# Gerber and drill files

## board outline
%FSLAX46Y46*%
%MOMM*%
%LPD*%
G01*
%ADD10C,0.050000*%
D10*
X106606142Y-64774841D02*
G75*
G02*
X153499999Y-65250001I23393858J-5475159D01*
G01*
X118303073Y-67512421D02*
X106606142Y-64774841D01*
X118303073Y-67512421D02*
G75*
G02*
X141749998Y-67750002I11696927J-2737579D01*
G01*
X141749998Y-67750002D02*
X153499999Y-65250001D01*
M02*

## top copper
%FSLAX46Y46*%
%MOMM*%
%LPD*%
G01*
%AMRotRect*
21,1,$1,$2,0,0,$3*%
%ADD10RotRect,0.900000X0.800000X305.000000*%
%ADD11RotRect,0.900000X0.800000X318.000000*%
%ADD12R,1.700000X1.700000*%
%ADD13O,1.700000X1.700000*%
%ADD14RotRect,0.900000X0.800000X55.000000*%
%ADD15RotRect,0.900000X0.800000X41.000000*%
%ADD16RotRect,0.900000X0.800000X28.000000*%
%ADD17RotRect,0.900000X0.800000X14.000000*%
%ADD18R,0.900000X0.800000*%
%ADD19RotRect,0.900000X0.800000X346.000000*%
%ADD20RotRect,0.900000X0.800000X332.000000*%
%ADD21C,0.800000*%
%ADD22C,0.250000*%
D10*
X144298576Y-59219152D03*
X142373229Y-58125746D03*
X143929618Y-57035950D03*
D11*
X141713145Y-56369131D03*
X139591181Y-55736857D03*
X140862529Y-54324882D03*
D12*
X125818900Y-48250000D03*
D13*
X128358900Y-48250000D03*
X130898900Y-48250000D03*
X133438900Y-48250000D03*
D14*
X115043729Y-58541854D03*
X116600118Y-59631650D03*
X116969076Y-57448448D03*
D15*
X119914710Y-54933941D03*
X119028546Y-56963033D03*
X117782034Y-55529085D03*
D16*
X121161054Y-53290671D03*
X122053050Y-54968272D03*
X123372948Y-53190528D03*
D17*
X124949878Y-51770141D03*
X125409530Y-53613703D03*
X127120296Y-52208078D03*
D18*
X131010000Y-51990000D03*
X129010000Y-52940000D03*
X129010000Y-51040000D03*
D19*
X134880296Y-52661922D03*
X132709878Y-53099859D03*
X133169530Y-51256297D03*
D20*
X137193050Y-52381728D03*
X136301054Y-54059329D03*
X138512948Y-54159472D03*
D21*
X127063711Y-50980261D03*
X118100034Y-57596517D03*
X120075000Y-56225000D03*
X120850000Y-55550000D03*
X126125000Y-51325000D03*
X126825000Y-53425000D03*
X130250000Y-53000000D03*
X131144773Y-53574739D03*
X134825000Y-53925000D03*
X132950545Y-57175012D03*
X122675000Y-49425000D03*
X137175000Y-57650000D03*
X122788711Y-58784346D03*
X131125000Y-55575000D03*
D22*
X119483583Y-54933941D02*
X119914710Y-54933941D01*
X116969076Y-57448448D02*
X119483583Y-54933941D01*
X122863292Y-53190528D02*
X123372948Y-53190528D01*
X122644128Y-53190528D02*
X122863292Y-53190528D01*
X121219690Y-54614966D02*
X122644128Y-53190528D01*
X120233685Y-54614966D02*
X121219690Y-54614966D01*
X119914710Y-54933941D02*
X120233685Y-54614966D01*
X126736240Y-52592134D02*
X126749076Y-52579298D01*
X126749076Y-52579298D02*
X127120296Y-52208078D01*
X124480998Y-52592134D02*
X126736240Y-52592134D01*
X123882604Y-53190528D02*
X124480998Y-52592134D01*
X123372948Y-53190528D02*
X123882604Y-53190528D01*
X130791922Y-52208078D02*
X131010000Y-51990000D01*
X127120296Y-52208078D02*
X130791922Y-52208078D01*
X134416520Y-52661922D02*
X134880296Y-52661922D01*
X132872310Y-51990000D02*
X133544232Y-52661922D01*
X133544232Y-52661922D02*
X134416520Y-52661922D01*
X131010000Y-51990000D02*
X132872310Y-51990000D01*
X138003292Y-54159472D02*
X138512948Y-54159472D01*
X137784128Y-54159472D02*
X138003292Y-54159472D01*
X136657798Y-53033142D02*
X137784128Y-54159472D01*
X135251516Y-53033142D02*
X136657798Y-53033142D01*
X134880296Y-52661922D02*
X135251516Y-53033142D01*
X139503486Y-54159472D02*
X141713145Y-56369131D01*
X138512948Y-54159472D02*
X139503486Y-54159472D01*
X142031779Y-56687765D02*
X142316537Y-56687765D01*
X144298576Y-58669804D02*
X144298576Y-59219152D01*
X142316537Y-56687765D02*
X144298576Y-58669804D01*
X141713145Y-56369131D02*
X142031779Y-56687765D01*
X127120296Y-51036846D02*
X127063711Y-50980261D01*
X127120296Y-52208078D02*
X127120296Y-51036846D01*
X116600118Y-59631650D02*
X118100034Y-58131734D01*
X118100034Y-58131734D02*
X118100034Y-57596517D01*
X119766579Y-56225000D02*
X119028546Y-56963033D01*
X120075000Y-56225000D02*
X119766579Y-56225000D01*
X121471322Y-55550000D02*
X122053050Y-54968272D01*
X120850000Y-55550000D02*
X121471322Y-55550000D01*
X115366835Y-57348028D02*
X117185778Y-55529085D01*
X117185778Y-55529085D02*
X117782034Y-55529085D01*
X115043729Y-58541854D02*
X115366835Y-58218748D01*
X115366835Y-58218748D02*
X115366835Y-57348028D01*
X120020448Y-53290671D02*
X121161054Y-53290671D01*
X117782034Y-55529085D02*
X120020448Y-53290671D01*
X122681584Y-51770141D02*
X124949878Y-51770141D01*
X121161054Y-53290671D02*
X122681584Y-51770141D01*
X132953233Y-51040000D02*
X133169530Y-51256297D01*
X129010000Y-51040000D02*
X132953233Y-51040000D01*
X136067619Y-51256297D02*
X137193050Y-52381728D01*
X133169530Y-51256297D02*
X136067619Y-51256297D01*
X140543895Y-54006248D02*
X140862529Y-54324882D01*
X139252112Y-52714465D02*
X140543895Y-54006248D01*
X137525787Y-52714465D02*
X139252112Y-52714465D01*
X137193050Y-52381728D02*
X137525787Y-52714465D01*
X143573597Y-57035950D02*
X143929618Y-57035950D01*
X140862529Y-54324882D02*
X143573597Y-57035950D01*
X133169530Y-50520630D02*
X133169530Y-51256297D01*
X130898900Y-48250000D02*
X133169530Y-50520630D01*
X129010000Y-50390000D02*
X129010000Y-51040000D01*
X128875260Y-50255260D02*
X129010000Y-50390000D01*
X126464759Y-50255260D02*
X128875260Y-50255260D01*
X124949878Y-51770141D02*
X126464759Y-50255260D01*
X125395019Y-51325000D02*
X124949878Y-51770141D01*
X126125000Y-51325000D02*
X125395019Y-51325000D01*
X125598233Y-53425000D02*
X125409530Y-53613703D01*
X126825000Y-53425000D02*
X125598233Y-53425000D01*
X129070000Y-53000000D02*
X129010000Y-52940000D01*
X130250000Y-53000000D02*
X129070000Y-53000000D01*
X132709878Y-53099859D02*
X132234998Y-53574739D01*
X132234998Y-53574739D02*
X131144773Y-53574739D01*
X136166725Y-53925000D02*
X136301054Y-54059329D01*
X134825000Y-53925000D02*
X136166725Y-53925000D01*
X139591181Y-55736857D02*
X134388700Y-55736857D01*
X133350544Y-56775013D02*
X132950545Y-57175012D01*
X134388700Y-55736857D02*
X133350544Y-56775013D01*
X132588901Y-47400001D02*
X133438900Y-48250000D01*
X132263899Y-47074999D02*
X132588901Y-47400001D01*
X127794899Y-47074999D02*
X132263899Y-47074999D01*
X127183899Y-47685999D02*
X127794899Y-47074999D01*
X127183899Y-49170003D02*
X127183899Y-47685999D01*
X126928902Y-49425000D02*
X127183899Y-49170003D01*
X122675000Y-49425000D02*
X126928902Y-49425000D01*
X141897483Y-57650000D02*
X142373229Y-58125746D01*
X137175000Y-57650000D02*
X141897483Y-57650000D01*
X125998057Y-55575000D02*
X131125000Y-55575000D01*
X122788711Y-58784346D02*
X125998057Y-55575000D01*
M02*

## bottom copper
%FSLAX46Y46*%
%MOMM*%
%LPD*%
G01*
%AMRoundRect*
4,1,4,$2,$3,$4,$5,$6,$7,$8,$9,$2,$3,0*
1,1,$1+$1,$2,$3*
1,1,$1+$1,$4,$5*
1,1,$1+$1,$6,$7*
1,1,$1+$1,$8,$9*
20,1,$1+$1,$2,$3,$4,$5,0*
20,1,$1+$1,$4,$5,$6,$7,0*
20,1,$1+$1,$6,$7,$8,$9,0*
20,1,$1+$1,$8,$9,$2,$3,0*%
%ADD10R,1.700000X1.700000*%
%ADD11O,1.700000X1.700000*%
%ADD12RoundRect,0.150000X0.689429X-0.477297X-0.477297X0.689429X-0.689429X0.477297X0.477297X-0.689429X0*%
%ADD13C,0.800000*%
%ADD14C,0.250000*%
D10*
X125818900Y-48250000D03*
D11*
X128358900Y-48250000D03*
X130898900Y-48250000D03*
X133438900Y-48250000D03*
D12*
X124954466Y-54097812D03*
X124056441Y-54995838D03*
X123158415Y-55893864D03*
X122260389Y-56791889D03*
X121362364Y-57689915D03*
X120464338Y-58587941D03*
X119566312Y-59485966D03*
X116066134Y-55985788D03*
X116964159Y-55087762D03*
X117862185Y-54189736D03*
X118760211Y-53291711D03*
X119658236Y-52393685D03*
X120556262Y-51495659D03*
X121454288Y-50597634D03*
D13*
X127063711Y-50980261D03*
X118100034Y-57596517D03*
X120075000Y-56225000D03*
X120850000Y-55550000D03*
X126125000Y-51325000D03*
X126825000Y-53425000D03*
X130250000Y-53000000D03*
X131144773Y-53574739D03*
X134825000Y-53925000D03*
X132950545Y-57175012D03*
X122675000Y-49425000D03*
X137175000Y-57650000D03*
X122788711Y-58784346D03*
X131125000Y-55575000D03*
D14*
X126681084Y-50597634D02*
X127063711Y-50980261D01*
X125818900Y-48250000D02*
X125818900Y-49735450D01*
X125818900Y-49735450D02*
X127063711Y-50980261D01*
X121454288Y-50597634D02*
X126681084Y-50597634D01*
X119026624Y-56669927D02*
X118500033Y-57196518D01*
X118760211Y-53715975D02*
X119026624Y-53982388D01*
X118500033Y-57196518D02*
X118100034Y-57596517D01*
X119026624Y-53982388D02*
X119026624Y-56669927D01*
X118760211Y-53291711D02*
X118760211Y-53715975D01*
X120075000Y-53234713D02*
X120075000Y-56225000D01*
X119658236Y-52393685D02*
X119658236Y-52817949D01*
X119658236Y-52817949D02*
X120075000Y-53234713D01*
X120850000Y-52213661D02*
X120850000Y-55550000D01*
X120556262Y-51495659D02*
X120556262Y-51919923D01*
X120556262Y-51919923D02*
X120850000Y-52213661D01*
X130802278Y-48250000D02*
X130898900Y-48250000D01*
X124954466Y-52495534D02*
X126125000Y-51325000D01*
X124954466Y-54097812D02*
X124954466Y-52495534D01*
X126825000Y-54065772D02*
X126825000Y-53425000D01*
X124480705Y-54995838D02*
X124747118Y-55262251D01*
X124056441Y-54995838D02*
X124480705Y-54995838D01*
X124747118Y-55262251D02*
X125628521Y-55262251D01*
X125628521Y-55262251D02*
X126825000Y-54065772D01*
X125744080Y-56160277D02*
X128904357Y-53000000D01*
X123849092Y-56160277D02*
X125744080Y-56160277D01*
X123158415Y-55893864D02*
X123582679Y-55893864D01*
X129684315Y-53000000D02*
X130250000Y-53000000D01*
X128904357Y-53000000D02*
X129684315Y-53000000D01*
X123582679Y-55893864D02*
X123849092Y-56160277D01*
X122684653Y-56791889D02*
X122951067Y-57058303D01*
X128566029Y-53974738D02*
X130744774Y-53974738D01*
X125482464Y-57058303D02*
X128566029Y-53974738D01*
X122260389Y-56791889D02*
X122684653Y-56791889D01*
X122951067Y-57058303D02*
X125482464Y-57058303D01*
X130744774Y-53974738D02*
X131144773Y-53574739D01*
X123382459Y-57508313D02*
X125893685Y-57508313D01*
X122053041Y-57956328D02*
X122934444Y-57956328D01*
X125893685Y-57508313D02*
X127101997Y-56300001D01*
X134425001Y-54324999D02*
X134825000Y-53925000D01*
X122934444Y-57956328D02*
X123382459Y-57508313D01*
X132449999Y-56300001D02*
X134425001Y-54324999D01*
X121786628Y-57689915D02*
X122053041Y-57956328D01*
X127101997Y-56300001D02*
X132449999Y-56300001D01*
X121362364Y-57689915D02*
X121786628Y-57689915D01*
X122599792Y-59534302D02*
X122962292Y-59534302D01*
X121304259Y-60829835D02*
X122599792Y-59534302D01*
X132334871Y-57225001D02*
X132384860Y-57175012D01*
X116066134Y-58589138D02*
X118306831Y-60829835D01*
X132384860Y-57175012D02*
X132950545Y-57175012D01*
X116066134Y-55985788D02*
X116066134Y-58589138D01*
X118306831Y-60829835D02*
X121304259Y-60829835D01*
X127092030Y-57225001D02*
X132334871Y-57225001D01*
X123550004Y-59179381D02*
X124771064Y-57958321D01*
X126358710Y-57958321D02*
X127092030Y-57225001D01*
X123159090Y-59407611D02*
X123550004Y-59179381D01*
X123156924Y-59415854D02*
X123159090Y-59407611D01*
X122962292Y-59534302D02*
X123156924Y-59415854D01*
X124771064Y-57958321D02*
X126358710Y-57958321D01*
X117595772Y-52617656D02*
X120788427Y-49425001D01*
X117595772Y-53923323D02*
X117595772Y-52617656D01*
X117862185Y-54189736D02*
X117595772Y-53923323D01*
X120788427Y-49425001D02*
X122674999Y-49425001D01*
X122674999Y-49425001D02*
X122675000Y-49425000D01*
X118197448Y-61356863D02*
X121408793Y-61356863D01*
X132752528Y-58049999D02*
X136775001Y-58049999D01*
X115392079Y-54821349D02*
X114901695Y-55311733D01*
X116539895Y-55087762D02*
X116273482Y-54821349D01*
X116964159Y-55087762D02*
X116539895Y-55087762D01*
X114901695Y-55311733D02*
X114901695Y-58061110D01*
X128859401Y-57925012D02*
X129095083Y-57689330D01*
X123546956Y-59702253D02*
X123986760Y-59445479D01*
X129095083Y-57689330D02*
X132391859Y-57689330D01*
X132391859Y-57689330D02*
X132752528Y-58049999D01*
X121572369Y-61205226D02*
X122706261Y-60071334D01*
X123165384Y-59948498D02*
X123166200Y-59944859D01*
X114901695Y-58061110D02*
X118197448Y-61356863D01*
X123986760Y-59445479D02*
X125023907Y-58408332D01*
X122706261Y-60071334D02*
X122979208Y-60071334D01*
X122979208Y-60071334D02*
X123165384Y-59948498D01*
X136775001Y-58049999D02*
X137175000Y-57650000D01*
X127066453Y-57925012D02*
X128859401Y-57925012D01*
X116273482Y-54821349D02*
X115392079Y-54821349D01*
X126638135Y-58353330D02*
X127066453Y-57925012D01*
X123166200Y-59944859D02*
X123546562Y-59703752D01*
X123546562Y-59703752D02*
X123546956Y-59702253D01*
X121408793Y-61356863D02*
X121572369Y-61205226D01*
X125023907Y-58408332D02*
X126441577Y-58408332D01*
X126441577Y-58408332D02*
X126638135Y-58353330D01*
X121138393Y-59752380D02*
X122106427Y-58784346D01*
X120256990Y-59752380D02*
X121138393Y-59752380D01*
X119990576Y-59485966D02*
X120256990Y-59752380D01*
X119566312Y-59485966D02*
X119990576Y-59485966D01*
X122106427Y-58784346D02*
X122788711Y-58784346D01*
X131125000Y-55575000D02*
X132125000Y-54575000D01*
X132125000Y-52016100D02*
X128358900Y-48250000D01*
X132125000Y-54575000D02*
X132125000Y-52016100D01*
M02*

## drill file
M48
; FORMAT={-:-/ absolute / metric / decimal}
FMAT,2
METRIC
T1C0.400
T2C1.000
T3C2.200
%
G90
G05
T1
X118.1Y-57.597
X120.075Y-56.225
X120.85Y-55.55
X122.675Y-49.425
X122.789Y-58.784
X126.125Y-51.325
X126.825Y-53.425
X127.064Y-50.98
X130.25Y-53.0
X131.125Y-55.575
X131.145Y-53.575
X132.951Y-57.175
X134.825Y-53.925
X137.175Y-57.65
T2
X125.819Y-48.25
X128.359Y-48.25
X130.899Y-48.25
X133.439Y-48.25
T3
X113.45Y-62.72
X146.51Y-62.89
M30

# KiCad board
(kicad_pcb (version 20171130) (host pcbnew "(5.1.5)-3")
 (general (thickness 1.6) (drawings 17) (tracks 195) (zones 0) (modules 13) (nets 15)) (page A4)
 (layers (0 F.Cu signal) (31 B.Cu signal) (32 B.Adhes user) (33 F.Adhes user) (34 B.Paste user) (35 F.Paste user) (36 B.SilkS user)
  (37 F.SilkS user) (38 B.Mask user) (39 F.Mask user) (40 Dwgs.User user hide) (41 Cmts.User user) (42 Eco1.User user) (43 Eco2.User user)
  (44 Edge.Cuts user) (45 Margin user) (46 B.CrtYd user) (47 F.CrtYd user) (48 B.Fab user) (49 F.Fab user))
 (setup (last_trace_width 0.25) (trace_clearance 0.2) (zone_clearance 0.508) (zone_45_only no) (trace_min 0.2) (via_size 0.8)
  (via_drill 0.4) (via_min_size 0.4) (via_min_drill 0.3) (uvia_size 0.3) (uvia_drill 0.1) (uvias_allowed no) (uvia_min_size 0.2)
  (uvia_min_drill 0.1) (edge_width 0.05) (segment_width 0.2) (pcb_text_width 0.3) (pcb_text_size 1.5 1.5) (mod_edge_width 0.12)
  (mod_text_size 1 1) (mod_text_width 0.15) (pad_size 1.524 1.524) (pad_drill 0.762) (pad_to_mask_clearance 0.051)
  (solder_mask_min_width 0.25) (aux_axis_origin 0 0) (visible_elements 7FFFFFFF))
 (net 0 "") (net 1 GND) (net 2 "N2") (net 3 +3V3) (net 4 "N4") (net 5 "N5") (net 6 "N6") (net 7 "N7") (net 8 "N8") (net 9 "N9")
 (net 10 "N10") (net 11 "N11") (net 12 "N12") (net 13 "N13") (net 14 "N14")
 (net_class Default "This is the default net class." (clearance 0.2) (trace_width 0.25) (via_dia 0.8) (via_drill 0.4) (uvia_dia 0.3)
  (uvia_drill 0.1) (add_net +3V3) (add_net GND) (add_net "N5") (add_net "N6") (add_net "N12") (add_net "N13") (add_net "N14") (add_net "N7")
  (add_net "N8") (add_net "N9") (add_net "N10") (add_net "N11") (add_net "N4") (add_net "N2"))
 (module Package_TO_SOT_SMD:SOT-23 (layer F.Cu) (at 143.725 58.4 305)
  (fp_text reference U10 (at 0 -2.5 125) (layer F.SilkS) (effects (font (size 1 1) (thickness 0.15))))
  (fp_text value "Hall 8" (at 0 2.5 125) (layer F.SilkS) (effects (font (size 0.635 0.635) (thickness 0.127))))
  (pad 3 smd rect (at 1 0 305) (size 0.9 0.8) (layers F.Cu F.Paste F.Mask) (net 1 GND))
  (pad 2 smd rect (at -1 0.95 305) (size 0.9 0.8) (layers F.Cu F.Paste F.Mask) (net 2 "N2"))
  (pad 1 smd rect (at -1 -0.95 305) (size 0.9 0.8) (layers F.Cu F.Paste F.Mask) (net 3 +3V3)))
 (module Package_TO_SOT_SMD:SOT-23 (layer F.Cu) (at 140.97 55.7 318)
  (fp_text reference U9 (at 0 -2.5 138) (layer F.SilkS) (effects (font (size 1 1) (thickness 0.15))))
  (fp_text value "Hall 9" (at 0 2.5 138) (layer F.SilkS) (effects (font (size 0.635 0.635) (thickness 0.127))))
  (pad 3 smd rect (at 1 0 318) (size 0.9 0.8) (layers F.Cu F.Paste F.Mask) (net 1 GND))
  (pad 2 smd rect (at -1 0.95 318) (size 0.9 0.8) (layers F.Cu F.Paste F.Mask) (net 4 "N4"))
  (pad 1 smd rect (at -1 -0.95 318) (size 0.9 0.8) (layers F.Cu F.Paste F.Mask) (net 3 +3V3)))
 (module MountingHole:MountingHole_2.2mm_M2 (layer F.Cu) (at 146.51 62.89)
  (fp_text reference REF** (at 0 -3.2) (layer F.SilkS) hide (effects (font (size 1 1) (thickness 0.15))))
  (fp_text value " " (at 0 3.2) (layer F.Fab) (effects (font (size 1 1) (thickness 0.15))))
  (pad 1 np_thru_hole circle (at 0 0) (size 2.2 2.2) (drill 2.2) (layers *.Cu *.Mask)))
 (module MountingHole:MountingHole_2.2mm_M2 (layer F.Cu) (at 113.45 62.72)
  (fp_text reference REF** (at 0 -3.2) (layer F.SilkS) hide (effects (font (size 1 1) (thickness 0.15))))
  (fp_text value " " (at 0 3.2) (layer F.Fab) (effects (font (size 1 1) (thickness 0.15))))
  (pad 1 np_thru_hole circle (at 0 0) (size 2.2 2.2) (drill 2.2) (layers *.Cu *.Mask)))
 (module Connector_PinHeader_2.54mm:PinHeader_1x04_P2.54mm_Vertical (layer F.Cu) (at 125.8189 48.25 90)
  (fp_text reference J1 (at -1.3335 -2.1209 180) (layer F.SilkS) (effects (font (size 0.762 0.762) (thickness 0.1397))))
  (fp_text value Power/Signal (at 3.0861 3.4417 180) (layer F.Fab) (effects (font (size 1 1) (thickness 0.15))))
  (pad 1 thru_hole rect (at 0 0 90) (size 1.7 1.7) (drill 1) (layers *.Cu *.Mask) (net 1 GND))
  (pad 2 thru_hole oval (at 0 2.54 90) (size 1.7 1.7) (drill 1) (layers *.Cu *.Mask) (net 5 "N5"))
  (pad 3 thru_hole oval (at 0 5.08 90) (size 1.7 1.7) (drill 1) (layers *.Cu *.Mask) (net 3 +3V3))
  (pad 4 thru_hole oval (at 0 7.62 90) (size 1.7 1.7) (drill 1) (layers *.Cu *.Mask) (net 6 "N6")))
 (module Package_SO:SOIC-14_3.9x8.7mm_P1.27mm (layer B.Cu) (at 120.5103 55.0418 135)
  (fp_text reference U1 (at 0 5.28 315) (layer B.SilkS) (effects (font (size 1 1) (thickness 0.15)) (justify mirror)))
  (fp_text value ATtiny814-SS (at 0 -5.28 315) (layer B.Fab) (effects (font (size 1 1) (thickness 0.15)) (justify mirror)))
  (pad 1 smd roundrect (at -2.475 3.81 135) (size 1.95 0.6) (layers B.Cu B.Paste B.Mask) (roundrect_rratio 0.25) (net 3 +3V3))
  (pad 2 smd roundrect (at -2.475 2.54 135) (size 1.95 0.6) (layers B.Cu B.Paste B.Mask) (roundrect_rratio 0.25) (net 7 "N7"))
  (pad 3 smd roundrect (at -2.475 1.27 135) (size 1.95 0.6) (layers B.Cu B.Paste B.Mask) (roundrect_rratio 0.25) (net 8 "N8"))
  (pad 4 smd roundrect (at -2.475 0 135) (size 1.95 0.6) (layers B.Cu B.Paste B.Mask) (roundrect_rratio 0.25) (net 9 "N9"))
  (pad 5 smd roundrect (at -2.475 -1.27 135) (size 1.95 0.6) (layers B.Cu B.Paste B.Mask) (roundrect_rratio 0.25) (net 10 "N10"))
  (pad 6 smd roundrect (at -2.475 -2.54 135) (size 1.95 0.6) (layers B.Cu B.Paste B.Mask) (roundrect_rratio 0.25) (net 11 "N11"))
  (pad 7 smd roundrect (at -2.475 -3.81 135) (size 1.95 0.6) (layers B.Cu B.Paste B.Mask) (roundrect_rratio 0.25) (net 5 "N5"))
  (pad 8 smd roundrect (at 2.475 -3.81 135) (size 1.95 0.6) (layers B.Cu B.Paste B.Mask) (roundrect_rratio 0.25) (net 4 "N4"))
  (pad 9 smd roundrect (at 2.475 -2.54 135) (size 1.95 0.6) (layers B.Cu B.Paste B.Mask) (roundrect_rratio 0.25) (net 2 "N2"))
  (pad 10 smd roundrect (at 2.475 -1.27 135) (size 1.95 0.6) (layers B.Cu B.Paste B.Mask) (roundrect_rratio 0.25) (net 6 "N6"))
  (pad 11 smd roundrect (at 2.475 0 135) (size 1.95 0.6) (layers B.Cu B.Paste B.Mask) (roundrect_rratio 0.25) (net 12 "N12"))
  (pad 12 smd roundrect (at 2.475 1.27 135) (size 1.95 0.6) (layers B.Cu B.Paste B.Mask) (roundrect_rratio 0.25) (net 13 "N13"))
  (pad 13 smd roundrect (at 2.475 2.54 135) (size 1.95 0.6) (layers B.Cu B.Paste B.Mask) (roundrect_rratio 0.25) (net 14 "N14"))
  (pad 14 smd roundrect (at 2.475 3.81 135) (size 1.95 0.6) (layers B.Cu B.Paste B.Mask) (roundrect_rratio 0.25) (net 1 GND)))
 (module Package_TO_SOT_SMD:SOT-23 (layer F.Cu) (at 116.3955 58.2676 55)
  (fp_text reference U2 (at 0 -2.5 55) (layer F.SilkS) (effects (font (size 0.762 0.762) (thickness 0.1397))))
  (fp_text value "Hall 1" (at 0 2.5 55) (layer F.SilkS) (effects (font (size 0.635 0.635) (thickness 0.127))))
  (pad 1 smd rect (at -1 -0.95 55) (size 0.9 0.8) (layers F.Cu F.Paste F.Mask) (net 3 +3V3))
  (pad 2 smd rect (at -1 0.95 55) (size 0.9 0.8) (layers F.Cu F.Paste F.Mask) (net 12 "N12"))
  (pad 3 smd rect (at 1 0 55) (size 0.9 0.8) (layers F.Cu F.Paste F.Mask) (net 1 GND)))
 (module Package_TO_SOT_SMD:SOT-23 (layer F.Cu) (at 119.16 55.59 41)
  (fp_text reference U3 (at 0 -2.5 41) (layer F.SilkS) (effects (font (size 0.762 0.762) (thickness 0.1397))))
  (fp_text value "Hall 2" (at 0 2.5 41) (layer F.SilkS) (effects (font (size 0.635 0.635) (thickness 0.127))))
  (pad 3 smd rect (at 1 0 41) (size 0.9 0.8) (layers F.Cu F.Paste F.Mask) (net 1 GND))
  (pad 2 smd rect (at -1 0.95 41) (size 0.9 0.8) (layers F.Cu F.Paste F.Mask) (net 13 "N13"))
  (pad 1 smd rect (at -1 -0.95 41) (size 0.9 0.8) (layers F.Cu F.Paste F.Mask) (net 3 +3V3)))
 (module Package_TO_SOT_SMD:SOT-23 (layer F.Cu) (at 122.49 53.66 28)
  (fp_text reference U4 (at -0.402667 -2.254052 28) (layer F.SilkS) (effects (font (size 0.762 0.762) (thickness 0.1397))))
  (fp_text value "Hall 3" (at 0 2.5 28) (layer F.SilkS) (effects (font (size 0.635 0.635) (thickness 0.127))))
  (pad 1 smd rect (at -1 -0.95 28) (size 0.9 0.8) (layers F.Cu F.Paste F.Mask) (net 3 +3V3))
  (pad 2 smd rect (at -1 0.95 28) (size 0.9 0.8) (layers F.Cu F.Paste F.Mask) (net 14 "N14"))
  (pad 3 smd rect (at 1 0 28) (size 0.9 0.8) (layers F.Cu F.Paste F.Mask) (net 1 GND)))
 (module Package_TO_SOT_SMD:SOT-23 (layer F.Cu) (at 126.15 52.45 14)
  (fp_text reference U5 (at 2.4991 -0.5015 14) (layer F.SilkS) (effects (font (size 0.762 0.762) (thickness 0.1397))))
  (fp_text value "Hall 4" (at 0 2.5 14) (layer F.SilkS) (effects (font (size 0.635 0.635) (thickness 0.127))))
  (pad 1 smd rect (at -1 -0.95 14) (size 0.9 0.8) (layers F.Cu F.Paste F.Mask) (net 3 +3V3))
  (pad 2 smd rect (at -1 0.95 14) (size 0.9 0.8) (layers F.Cu F.Paste F.Mask) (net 7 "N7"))
  (pad 3 smd rect (at 1 0 14) (size 0.9 0.8) (layers F.Cu F.Paste F.Mask) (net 1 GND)))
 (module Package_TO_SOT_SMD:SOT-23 (layer F.Cu) (at 130.01 51.99)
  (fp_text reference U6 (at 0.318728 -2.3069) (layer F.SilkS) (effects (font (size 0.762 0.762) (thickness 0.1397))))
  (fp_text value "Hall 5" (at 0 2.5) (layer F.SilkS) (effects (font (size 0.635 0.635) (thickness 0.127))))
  (pad 3 smd rect (at 1 0) (size 0.9 0.8) (layers F.Cu F.Paste F.Mask) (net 1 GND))
  (pad 2 smd rect (at -1 0.95) (size 0.9 0.8) (layers F.Cu F.Paste F.Mask) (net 8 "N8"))
  (pad 1 smd rect (at -1 -0.95) (size 0.9 0.8) (layers F.Cu F.Paste F.Mask) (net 3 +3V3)))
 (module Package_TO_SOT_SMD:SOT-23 (layer F.Cu) (at 133.91 52.42 346)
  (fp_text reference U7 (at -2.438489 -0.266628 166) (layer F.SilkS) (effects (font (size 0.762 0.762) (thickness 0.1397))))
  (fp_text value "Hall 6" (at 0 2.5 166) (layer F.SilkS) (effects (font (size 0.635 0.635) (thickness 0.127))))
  (pad 3 smd rect (at 1 0 346) (size 0.9 0.8) (layers F.Cu F.Paste F.Mask) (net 1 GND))
  (pad 2 smd rect (at -1 0.95 346) (size 0.9 0.8) (layers F.Cu F.Paste F.Mask) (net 9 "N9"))
  (pad 1 smd rect (at -1 -0.95 346) (size 0.9 0.8) (layers F.Cu F.Paste F.Mask) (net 3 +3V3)))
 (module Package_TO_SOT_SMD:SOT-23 (layer F.Cu) (at 137.63 53.69 332)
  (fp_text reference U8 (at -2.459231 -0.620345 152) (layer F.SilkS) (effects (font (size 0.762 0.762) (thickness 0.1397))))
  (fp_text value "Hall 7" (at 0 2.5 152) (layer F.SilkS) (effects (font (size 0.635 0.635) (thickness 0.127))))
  (pad 1 smd rect (at -1 -0.95 332) (size 0.9 0.8) (layers F.Cu F.Paste F.Mask) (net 3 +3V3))
  (pad 2 smd rect (at -1 0.95 332) (size 0.9 0.8) (layers F.Cu F.Paste F.Mask) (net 10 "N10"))
  (pad 3 smd rect (at 1 0 332) (size 0.9 0.8) (layers F.Cu F.Paste F.Mask) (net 1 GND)))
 (gr_arc (start 130 70.25) (end 153.499999 65.250001) (angle -154.8159682) (layer Edge.Cuts) (width 0.05))
 (gr_line (start 118.303073 67.512421) (end 106.606142 64.774841) (layer Edge.Cuts) (width 0.05))
 (gr_arc (start 130 70.25) (end 141.749998 67.750002) (angle -154.8159719) (layer Edge.Cuts) (width 0.05))
 (gr_line (start 141.749998 67.750002) (end 153.499999 65.250001) (layer Edge.Cuts) (width 0.05))
 (segment (start 119.483583 54.933941) (end 119.91471 54.933941) (width 0.25) (layer F.Cu) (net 1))
 (segment (start 116.969076 57.448448) (end 119.483583 54.933941) (width 0.25) (layer F.Cu) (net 1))
 (segment (start 122.863292 53.190528) (end 123.372948 53.190528) (width 0.25) (layer F.Cu) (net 1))
 (segment (start 122.644128 53.190528) (end 122.863292 53.190528) (width 0.25) (layer F.Cu) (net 1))
 (segment (start 121.21969 54.614966) (end 122.644128 53.190528) (width 0.25) (layer F.Cu) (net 1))
 (segment (start 120.233685 54.614966) (end 121.21969 54.614966) (width 0.25) (layer F.Cu) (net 1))
 (segment (start 119.91471 54.933941) (end 120.233685 54.614966) (width 0.25) (layer F.Cu) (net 1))
 (segment (start 126.73624 52.592134) (end 126.749076 52.579298) (width 0.25) (layer F.Cu) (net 1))
 (segment (start 126.749076 52.579298) (end 127.120296 52.208078) (width 0.25) (layer F.Cu) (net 1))
 (segment (start 124.480998 52.592134) (end 126.73624 52.592134) (width 0.25) (layer F.Cu) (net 1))
 (segment (start 123.882604 53.190528) (end 124.480998 52.592134) (width 0.25) (layer F.Cu) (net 1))
 (segment (start 123.372948 53.190528) (end 123.882604 53.190528) (width 0.25) (layer F.Cu) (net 1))
 (segment (start 130.791922 52.208078) (end 131.01 51.99) (width 0.25) (layer F.Cu) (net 1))
 (segment (start 127.120296 52.208078) (end 130.791922 52.208078) (width 0.25) (layer F.Cu) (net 1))
 (segment (start 134.41652 52.661922) (end 134.880296 52.661922) (width 0.25) (layer F.Cu) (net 1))
 (segment (start 132.87231 51.99) (end 133.544232 52.661922) (width 0.25) (layer F.Cu) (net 1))
 (segment (start 133.544232 52.661922) (end 134.41652 52.661922) (width 0.25) (layer F.Cu) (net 1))
 (segment (start 131.01 51.99) (end 132.87231 51.99) (width 0.25) (layer F.Cu) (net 1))
 (segment (start 138.003292 54.159472) (end 138.512948 54.159472) (width 0.25) (layer F.Cu) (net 1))
 (segment (start 137.784128 54.159472) (end 138.003292 54.159472) (width 0.25) (layer F.Cu) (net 1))
 (segment (start 136.657798 53.033142) (end 137.784128 54.159472) (width 0.25) (layer F.Cu) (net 1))
 (segment (start 135.251516 53.033142) (end 136.657798 53.033142) (width 0.25) (layer F.Cu) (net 1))
 (segment (start 134.880296 52.661922) (end 135.251516 53.033142) (width 0.25) (layer F.Cu) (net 1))
 (segment (start 139.503486 54.159472) (end 141.713145 56.369131) (width 0.25) (layer F.Cu) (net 1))
 (segment (start 138.512948 54.159472) (end 139.503486 54.159472) (width 0.25) (layer F.Cu) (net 1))
 (segment (start 142.031779 56.687765) (end 142.316537 56.687765) (width 0.25) (layer F.Cu) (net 1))
 (segment (start 144.298576 58.669804) (end 144.298576 59.219152) (width 0.25) (layer F.Cu) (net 1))
 (segment (start 142.316537 56.687765) (end 144.298576 58.669804) (width 0.25) (layer F.Cu) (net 1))
 (segment (start 141.713145 56.369131) (end 142.031779 56.687765) (width 0.25) (layer F.Cu) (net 1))
 (segment (start 126.681084 50.597634) (end 127.063711 50.980261) (width 0.25) (layer B.Cu) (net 1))
 (segment (start 125.8189 48.25) (end 125.8189 49.73545) (width 0.25) (layer B.Cu) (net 1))
 (via (at 127.063711 50.980261) (size 0.8) (drill 0.4) (layers F.Cu B.Cu) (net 1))
 (segment (start 125.8189 49.73545) (end 127.063711 50.980261) (width 0.25) (layer B.Cu) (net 1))
 (segment (start 121.454288 50.597634) (end 126.681084 50.597634) (width 0.25) (layer B.Cu) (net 1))
 (segment (start 127.120296 51.036846) (end 127.063711 50.980261) (width 0.25) (layer F.Cu) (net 1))
 (segment (start 127.120296 52.208078) (end 127.120296 51.036846) (width 0.25) (layer F.Cu) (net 1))
 (segment (start 116.600118 59.63165) (end 118.100034 58.131734) (width 0.25) (layer F.Cu) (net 12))
 (via (at 118.100034 57.596517) (size 0.8) (drill 0.4) (layers F.Cu B.Cu) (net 12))
 (segment (start 118.100034 58.131734) (end 118.100034 57.596517) (width 0.25) (layer F.Cu) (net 12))
 (segment (start 119.026624 56.669927) (end 118.500033 57.196518) (width 0.25) (layer B.Cu) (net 12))
 (segment (start 118.760211 53.715975) (end 119.026624 53.982388) (width 0.25) (layer B.Cu) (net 12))
 (segment (start 118.500033 57.196518) (end 118.100034 57.596517) (width 0.25) (layer B.Cu) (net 12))
 (segment (start 119.026624 53.982388) (end 119.026624 56.669927) (width 0.25) (layer B.Cu) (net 12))
 (segment (start 118.760211 53.291711) (end 118.760211 53.715975) (width 0.25) (layer B.Cu) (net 12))
 (via (at 120.075 56.225) (size 0.8) (drill 0.4) (layers F.Cu B.Cu) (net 13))
 (segment (start 120.075 53.234713) (end 120.075 56.225) (width 0.25) (layer B.Cu) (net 13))
 (segment (start 119.658236 52.393685) (end 119.658236 52.817949) (width 0.25) (layer B.Cu) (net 13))
 (segment (start 119.658236 52.817949) (end 120.075 53.234713) (width 0.25) (layer B.Cu) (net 13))
 (segment (start 119.766579 56.225) (end 119.028546 56.963033) (width 0.25) (layer F.Cu) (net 13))
 (segment (start 120.075 56.225) (end 119.766579 56.225) (width 0.25) (layer F.Cu) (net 13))
 (segment (start 120.85 52.213661) (end 120.85 55.55) (width 0.25) (layer B.Cu) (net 14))
 (via (at 120.85 55.55) (size 0.8) (drill 0.4) (layers F.Cu B.Cu) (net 14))
 (segment (start 120.556262 51.495659) (end 120.556262 51.919923) (width 0.25) (layer B.Cu) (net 14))
 (segment (start 120.556262 51.919923) (end 120.85 52.213661) (width 0.25) (layer B.Cu) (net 14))
 (segment (start 121.471322 55.55) (end 122.05305 54.968272) (width 0.25) (layer F.Cu) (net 14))
 (segment (start 120.85 55.55) (end 121.471322 55.55) (width 0.25) (layer F.Cu) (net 14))
 (segment (start 115.366835 57.348028) (end 117.185778 55.529085) (width 0.25) (layer F.Cu) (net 3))
 (segment (start 117.185778 55.529085) (end 117.782034 55.529085) (width 0.25) (layer F.Cu) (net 3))
 (segment (start 115.043729 58.541854) (end 115.366835 58.218748) (width 0.25) (layer F.Cu) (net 3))
 (segment (start 115.366835 58.218748) (end 115.366835 57.348028) (width 0.25) (layer F.Cu) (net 3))
 (segment (start 120.020448 53.290671) (end 121.161054 53.290671) (width 0.25) (layer F.Cu) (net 3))
 (segment (start 117.782034 55.529085) (end 120.020448 53.290671) (width 0.25) (layer F.Cu) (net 3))
 (segment (start 122.681584 51.770141) (end 124.949878 51.770141) (width 0.25) (layer F.Cu) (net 3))
 (segment (start 121.161054 53.290671) (end 122.681584 51.770141) (width 0.25) (layer F.Cu) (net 3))
 (segment (start 132.953233 51.04) (end 133.16953 51.256297) (width 0.25) (layer F.Cu) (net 3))
 (segment (start 129.01 51.04) (end 132.953233 51.04) (width 0.25) (layer F.Cu) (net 3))
 (segment (start 136.067619 51.256297) (end 137.19305 52.381728) (width 0.25) (layer F.Cu) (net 3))
 (segment (start 133.16953 51.256297) (end 136.067619 51.256297) (width 0.25) (layer F.Cu) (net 3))
 (segment (start 140.543895 54.006248) (end 140.862529 54.324882) (width 0.25) (layer F.Cu) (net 3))
 (segment (start 139.252112 52.714465) (end 140.543895 54.006248) (width 0.25) (layer F.Cu) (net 3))
 (segment (start 137.525787 52.714465) (end 139.252112 52.714465) (width 0.25) (layer F.Cu) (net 3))
 (segment (start 137.19305 52.381728) (end 137.525787 52.714465) (width 0.25) (layer F.Cu) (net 3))
 (segment (start 143.573597 57.03595) (end 143.929618 57.03595) (width 0.25) (layer F.Cu) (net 3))
 (segment (start 140.862529 54.324882) (end 143.573597 57.03595) (width 0.25) (layer F.Cu) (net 3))
 (segment (start 130.802278 48.25) (end 130.8989 48.25) (width 0.25) (layer B.Cu) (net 3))
 (segment (start 133.16953 50.52063) (end 133.16953 51.256297) (width 0.25) (layer F.Cu) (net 3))
 (segment (start 130.8989 48.25) (end 133.16953 50.52063) (width 0.25) (layer F.Cu) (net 3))
 (via (at 126.125 51.325) (size 0.8) (drill 0.4) (layers F.Cu B.Cu) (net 3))
 (segment (start 124.954466 52.495534) (end 126.125 51.325) (width 0.25) (layer B.Cu) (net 3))
 (segment (start 124.954466 54.097812) (end 124.954466 52.495534) (width 0.25) (layer B.Cu) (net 3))
 (segment (start 129.01 50.39) (end 129.01 51.04) (width 0.25) (layer F.Cu) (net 3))
 (segment (start 128.87526 50.25526) (end 129.01 50.39) (width 0.25) (layer F.Cu) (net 3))
 (segment (start 126.464759 50.25526) (end 128.87526 50.25526) (width 0.25) (layer F.Cu) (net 3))
 (segment (start 124.949878 51.770141) (end 126.464759 50.25526) (width 0.25) (layer F.Cu) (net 3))
 (segment (start 125.395019 51.325) (end 124.949878 51.770141) (width 0.25) (layer F.Cu) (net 3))
 (segment (start 126.125 51.325) (end 125.395019 51.325) (width 0.25) (layer F.Cu) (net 3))
 (segment (start 126.825 54.065772) (end 126.825 53.425) (width 0.25) (layer B.Cu) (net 7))
 (via (at 126.825 53.425) (size 0.8) (drill 0.4) (layers F.Cu B.Cu) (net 7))
 (segment (start 124.480705 54.995838) (end 124.747118 55.262251) (width 0.25) (layer B.Cu) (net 7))
 (segment (start 124.056441 54.995838) (end 124.480705 54.995838) (width 0.25) (layer B.Cu) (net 7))
 (segment (start 124.747118 55.262251) (end 125.628521 55.262251) (width 0.25) (layer B.Cu) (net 7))
 (segment (start 125.628521 55.262251) (end 126.825 54.065772) (width 0.25) (layer B.Cu) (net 7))
 (segment (start 125.598233 53.425) (end 125.40953 53.613703) (width 0.25) (layer F.Cu) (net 7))
 (segment (start 126.825 53.425) (end 125.598233 53.425) (width 0.25) (layer F.Cu) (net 7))
 (via (at 130.25 53) (size 0.8) (drill 0.4) (layers F.Cu B.Cu) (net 8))
 (segment (start 129.07 53) (end 129.01 52.94) (width 0.25) (layer F.Cu) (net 8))
 (segment (start 130.25 53) (end 129.07 53) (width 0.25) (layer F.Cu) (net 8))
 (segment (start 125.74408 56.160277) (end 128.904357 53) (width 0.25) (layer B.Cu) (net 8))
 (segment (start 123.849092 56.160277) (end 125.74408 56.160277) (width 0.25) (layer B.Cu) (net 8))
 (segment (start 123.158415 55.893864) (end 123.582679 55.893864) (width 0.25) (layer B.Cu) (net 8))
 (segment (start 129.684315 53) (end 130.25 53) (width 0.25) (layer B.Cu) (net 8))
 (segment (start 128.904357 53) (end 129.684315 53) (width 0.25) (layer B.Cu) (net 8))
 (segment (start 123.582679 55.893864) (end 123.849092 56.160277) (width 0.25) (layer B.Cu) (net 8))
 (segment (start 122.684653 56.791889) (end 122.951067 57.058303) (width 0.25) (layer B.Cu) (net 9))
 (segment (start 128.566029 53.974738) (end 130.744774 53.974738) (width 0.25) (layer B.Cu) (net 9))
 (segment (start 132.709878 53.099859) (end 132.234998 53.574739) (width 0.25) (layer F.Cu) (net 9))
 (segment (start 125.482464 57.058303) (end 128.566029 53.974738) (width 0.25) (layer B.Cu) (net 9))
 (via (at 131.144773 53.574739) (size 0.8) (drill 0.4) (layers F.Cu B.Cu) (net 9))
 (segment (start 122.260389 56.791889) (end 122.684653 56.791889) (width 0.25) (layer B.Cu) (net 9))
 (segment (start 132.234998 53.574739) (end 131.144773 53.574739) (width 0.25) (layer F.Cu) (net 9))
 (segment (start 122.951067 57.058303) (end 125.482464 57.058303) (width 0.25) (layer B.Cu) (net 9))
 (segment (start 130.744774 53.974738) (end 131.144773 53.574739) (width 0.25) (layer B.Cu) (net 9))
 (via (at 134.825 53.925) (size 0.8) (drill 0.4) (layers F.Cu B.Cu) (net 10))
 (segment (start 136.166725 53.925) (end 136.301054 54.059329) (width 0.25) (layer F.Cu) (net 10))
 (segment (start 134.825 53.925) (end 136.166725 53.925) (width 0.25) (layer F.Cu) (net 10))
 (segment (start 123.382459 57.508313) (end 125.893685 57.508313) (width 0.25) (layer B.Cu) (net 10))
 (segment (start 122.053041 57.956328) (end 122.934444 57.956328) (width 0.25) (layer B.Cu) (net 10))
 (segment (start 125.893685 57.508313) (end 127.101997 56.300001) (width 0.25) (layer B.Cu) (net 10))
 (segment (start 134.425001 54.324999) (end 134.825 53.925) (width 0.25) (layer B.Cu) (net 10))
 (segment (start 122.934444 57.956328) (end 123.382459 57.508313) (width 0.25) (layer B.Cu) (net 10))
 (segment (start 132.449999 56.300001) (end 134.425001 54.324999) (width 0.25) (layer B.Cu) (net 10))
 (segment (start 121.786628 57.689915) (end 122.053041 57.956328) (width 0.25) (layer B.Cu) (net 10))
 (segment (start 127.101997 56.300001) (end 132.449999 56.300001) (width 0.25) (layer B.Cu) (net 10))
 (segment (start 121.362364 57.689915) (end 121.786628 57.689915) (width 0.25) (layer B.Cu) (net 10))
 (segment (start 139.591181 55.736857) (end 134.3887 55.736857) (width 0.25) (layer F.Cu) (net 4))
 (segment (start 133.350544 56.775013) (end 132.950545 57.175012) (width 0.25) (layer F.Cu) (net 4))
 (segment (start 134.3887 55.736857) (end 133.350544 56.775013) (width 0.25) (layer F.Cu) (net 4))
 (via (at 132.950545 57.175012) (size 0.8) (drill 0.4) (layers F.Cu B.Cu) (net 4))
 (segment (start 122.599792 59.534302) (end 122.962292 59.534302) (width 0.25) (layer B.Cu) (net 4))
 (segment (start 121.304259 60.829835) (end 122.599792 59.534302) (width 0.25) (layer B.Cu) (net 4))
 (segment (start 132.334871 57.225001) (end 132.38486 57.175012) (width 0.25) (layer B.Cu) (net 4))
 (segment (start 116.066134 58.589138) (end 118.306831 60.829835) (width 0.25) (layer B.Cu) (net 4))
 (segment (start 132.38486 57.175012) (end 132.950545 57.175012) (width 0.25) (layer B.Cu) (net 4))
 (segment (start 116.066134 55.985788) (end 116.066134 58.589138) (width 0.25) (layer B.Cu) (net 4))
 (segment (start 118.306831 60.829835) (end 121.304259 60.829835) (width 0.25) (layer B.Cu) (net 4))
 (segment (start 127.09203 57.225001) (end 132.334871 57.225001) (width 0.25) (layer B.Cu) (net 4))
 (segment (start 123.550004 59.179381) (end 124.771064 57.958321) (width 0.25) (layer B.Cu) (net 4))
 (segment (start 126.35871 57.958321) (end 127.09203 57.225001) (width 0.25) (layer B.Cu) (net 4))
 (segment (start 123.15909 59.407611) (end 123.550004 59.179381) (width 0.25) (layer B.Cu) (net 4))
 (segment (start 123.156924 59.415854) (end 123.15909 59.407611) (width 0.25) (layer B.Cu) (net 4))
 (segment (start 122.962292 59.534302) (end 123.156924 59.415854) (width 0.25) (layer B.Cu) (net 4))
 (segment (start 124.771064 57.958321) (end 126.35871 57.958321) (width 0.25) (layer B.Cu) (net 4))
 (segment (start 117.595772 52.617656) (end 120.788427 49.425001) (width 0.25) (layer B.Cu) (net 6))
 (segment (start 117.595772 53.923323) (end 117.595772 52.617656) (width 0.25) (layer B.Cu) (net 6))
 (segment (start 117.862185 54.189736) (end 117.595772 53.923323) (width 0.25) (layer B.Cu) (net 6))
 (via (at 122.675 49.425) (size 0.8) (drill 0.4) (layers F.Cu B.Cu) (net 6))
 (segment (start 120.788427 49.425001) (end 122.674999 49.425001) (width 0.25) (layer B.Cu) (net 6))
 (segment (start 122.674999 49.425001) (end 122.675 49.425) (width 0.25) (layer B.Cu) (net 6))
 (segment (start 132.588901 47.400001) (end 133.4389 48.25) (width 0.25) (layer F.Cu) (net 6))
 (segment (start 132.263899 47.074999) (end 132.588901 47.400001) (width 0.25) (layer F.Cu) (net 6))
 (segment (start 127.794899 47.074999) (end 132.263899 47.074999) (width 0.25) (layer F.Cu) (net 6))
 (segment (start 127.183899 47.685999) (end 127.794899 47.074999) (width 0.25) (layer F.Cu) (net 6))
 (segment (start 127.183899 49.170003) (end 127.183899 47.685999) (width 0.25) (layer F.Cu) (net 6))
 (segment (start 126.928902 49.425) (end 127.183899 49.170003) (width 0.25) (layer F.Cu) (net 6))
 (segment (start 122.675 49.425) (end 126.928902 49.425) (width 0.25) (layer F.Cu) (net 6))
 (via (at 137.175 57.65) (size 0.8) (drill 0.4) (layers F.Cu B.Cu) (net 2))
 (segment (start 141.897483 57.65) (end 142.373229 58.125746) (width 0.25) (layer F.Cu) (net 2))
 (segment (start 137.175 57.65) (end 141.897483 57.65) (width 0.25) (layer F.Cu) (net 2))
 (segment (start 118.197448 61.356863) (end 121.408793 61.356863) (width 0.25) (layer B.Cu) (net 2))
 (segment (start 132.752528 58.049999) (end 136.775001 58.049999) (width 0.25) (layer B.Cu) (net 2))
 (segment (start 115.392079 54.821349) (end 114.901695 55.311733) (width 0.25) (layer B.Cu) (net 2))
 (segment (start 116.539895 55.087762) (end 116.273482 54.821349) (width 0.25) (layer B.Cu) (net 2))
 (segment (start 116.964159 55.087762) (end 116.539895 55.087762) (width 0.25) (layer B.Cu) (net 2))
 (segment (start 114.901695 55.311733) (end 114.901695 58.06111) (width 0.25) (layer B.Cu) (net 2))
 (segment (start 128.859401 57.925012) (end 129.095083 57.68933) (width 0.25) (layer B.Cu) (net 2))
 (segment (start 123.546956 59.702253) (end 123.98676 59.445479) (width 0.25) (layer B.Cu) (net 2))
 (segment (start 129.095083 57.68933) (end 132.391859 57.68933) (width 0.25) (layer B.Cu) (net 2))
 (segment (start 132.391859 57.68933) (end 132.752528 58.049999) (width 0.25) (layer B.Cu) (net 2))
 (segment (start 121.572369 61.205226) (end 122.706261 60.071334) (width 0.25) (layer B.Cu) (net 2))
 (segment (start 123.165384 59.948498) (end 123.1662 59.944859) (width 0.25) (layer B.Cu) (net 2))
 (segment (start 114.901695 58.06111) (end 118.197448 61.356863) (width 0.25) (layer B.Cu) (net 2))
 (segment (start 123.98676 59.445479) (end 125.023907 58.408332) (width 0.25) (layer B.Cu) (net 2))
 (segment (start 122.706261 60.071334) (end 122.979208 60.071334) (width 0.25) (layer B.Cu) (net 2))
 (segment (start 122.979208 60.071334) (end 123.165384 59.948498) (width 0.25) (layer B.Cu) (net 2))
 (segment (start 136.775001 58.049999) (end 137.175 57.65) (width 0.25) (layer B.Cu) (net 2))
 (segment (start 127.066453 57.925012) (end 128.859401 57.925012) (width 0.25) (layer B.Cu) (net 2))
 (segment (start 116.273482 54.821349) (end 115.392079 54.821349) (width 0.25) (layer B.Cu) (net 2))
 (segment (start 126.638135 58.35333) (end 127.066453 57.925012) (width 0.25) (layer B.Cu) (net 2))
 (segment (start 123.1662 59.944859) (end 123.546562 59.703752) (width 0.25) (layer B.Cu) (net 2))
 (segment (start 123.546562 59.703752) (end 123.546956 59.702253) (width 0.25) (layer B.Cu) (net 2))
 (segment (start 121.408793 61.356863) (end 121.572369 61.205226) (width 0.25) (layer B.Cu) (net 2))
 (segment (start 125.023907 58.408332) (end 126.441577 58.408332) (width 0.25) (layer B.Cu) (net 2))
 (segment (start 126.441577 58.408332) (end 126.638135 58.35333) (width 0.25) (layer B.Cu) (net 2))
 (segment (start 121.138393 59.75238) (end 122.106427 58.784346) (width 0.25) (layer B.Cu) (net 5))
 (segment (start 120.25699 59.75238) (end 121.138393 59.75238) (width 0.25) (layer B.Cu) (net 5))
 (segment (start 119.990576 59.485966) (end 120.25699 59.75238) (width 0.25) (layer B.Cu) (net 5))
 (segment (start 119.566312 59.485966) (end 119.990576 59.485966) (width 0.25) (layer B.Cu) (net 5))
 (via (at 122.788711 58.784346) (size 0.8) (drill 0.4) (layers F.Cu B.Cu) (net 5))
 (segment (start 122.106427 58.784346) (end 122.788711 58.784346) (width 0.25) (layer B.Cu) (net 5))
 (segment (start 125.998057 55.575) (end 131.125 55.575) (width 0.25) (layer F.Cu) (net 5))
 (segment (start 122.788711 58.784346) (end 125.998057 55.575) (width 0.25) (layer F.Cu) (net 5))
 (via (at 131.125 55.575) (size 0.8) (drill 0.4) (layers F.Cu B.Cu) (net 5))
 (segment (start 131.125 55.575) (end 132.125 54.575) (width 0.25) (layer B.Cu) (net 5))
 (segment (start 132.125 52.0161) (end 128.3589 48.25) (width 0.25) (layer B.Cu) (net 5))
 (segment (start 132.125 54.575) (end 132.125 52.0161) (width 0.25) (layer B.Cu) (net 5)))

